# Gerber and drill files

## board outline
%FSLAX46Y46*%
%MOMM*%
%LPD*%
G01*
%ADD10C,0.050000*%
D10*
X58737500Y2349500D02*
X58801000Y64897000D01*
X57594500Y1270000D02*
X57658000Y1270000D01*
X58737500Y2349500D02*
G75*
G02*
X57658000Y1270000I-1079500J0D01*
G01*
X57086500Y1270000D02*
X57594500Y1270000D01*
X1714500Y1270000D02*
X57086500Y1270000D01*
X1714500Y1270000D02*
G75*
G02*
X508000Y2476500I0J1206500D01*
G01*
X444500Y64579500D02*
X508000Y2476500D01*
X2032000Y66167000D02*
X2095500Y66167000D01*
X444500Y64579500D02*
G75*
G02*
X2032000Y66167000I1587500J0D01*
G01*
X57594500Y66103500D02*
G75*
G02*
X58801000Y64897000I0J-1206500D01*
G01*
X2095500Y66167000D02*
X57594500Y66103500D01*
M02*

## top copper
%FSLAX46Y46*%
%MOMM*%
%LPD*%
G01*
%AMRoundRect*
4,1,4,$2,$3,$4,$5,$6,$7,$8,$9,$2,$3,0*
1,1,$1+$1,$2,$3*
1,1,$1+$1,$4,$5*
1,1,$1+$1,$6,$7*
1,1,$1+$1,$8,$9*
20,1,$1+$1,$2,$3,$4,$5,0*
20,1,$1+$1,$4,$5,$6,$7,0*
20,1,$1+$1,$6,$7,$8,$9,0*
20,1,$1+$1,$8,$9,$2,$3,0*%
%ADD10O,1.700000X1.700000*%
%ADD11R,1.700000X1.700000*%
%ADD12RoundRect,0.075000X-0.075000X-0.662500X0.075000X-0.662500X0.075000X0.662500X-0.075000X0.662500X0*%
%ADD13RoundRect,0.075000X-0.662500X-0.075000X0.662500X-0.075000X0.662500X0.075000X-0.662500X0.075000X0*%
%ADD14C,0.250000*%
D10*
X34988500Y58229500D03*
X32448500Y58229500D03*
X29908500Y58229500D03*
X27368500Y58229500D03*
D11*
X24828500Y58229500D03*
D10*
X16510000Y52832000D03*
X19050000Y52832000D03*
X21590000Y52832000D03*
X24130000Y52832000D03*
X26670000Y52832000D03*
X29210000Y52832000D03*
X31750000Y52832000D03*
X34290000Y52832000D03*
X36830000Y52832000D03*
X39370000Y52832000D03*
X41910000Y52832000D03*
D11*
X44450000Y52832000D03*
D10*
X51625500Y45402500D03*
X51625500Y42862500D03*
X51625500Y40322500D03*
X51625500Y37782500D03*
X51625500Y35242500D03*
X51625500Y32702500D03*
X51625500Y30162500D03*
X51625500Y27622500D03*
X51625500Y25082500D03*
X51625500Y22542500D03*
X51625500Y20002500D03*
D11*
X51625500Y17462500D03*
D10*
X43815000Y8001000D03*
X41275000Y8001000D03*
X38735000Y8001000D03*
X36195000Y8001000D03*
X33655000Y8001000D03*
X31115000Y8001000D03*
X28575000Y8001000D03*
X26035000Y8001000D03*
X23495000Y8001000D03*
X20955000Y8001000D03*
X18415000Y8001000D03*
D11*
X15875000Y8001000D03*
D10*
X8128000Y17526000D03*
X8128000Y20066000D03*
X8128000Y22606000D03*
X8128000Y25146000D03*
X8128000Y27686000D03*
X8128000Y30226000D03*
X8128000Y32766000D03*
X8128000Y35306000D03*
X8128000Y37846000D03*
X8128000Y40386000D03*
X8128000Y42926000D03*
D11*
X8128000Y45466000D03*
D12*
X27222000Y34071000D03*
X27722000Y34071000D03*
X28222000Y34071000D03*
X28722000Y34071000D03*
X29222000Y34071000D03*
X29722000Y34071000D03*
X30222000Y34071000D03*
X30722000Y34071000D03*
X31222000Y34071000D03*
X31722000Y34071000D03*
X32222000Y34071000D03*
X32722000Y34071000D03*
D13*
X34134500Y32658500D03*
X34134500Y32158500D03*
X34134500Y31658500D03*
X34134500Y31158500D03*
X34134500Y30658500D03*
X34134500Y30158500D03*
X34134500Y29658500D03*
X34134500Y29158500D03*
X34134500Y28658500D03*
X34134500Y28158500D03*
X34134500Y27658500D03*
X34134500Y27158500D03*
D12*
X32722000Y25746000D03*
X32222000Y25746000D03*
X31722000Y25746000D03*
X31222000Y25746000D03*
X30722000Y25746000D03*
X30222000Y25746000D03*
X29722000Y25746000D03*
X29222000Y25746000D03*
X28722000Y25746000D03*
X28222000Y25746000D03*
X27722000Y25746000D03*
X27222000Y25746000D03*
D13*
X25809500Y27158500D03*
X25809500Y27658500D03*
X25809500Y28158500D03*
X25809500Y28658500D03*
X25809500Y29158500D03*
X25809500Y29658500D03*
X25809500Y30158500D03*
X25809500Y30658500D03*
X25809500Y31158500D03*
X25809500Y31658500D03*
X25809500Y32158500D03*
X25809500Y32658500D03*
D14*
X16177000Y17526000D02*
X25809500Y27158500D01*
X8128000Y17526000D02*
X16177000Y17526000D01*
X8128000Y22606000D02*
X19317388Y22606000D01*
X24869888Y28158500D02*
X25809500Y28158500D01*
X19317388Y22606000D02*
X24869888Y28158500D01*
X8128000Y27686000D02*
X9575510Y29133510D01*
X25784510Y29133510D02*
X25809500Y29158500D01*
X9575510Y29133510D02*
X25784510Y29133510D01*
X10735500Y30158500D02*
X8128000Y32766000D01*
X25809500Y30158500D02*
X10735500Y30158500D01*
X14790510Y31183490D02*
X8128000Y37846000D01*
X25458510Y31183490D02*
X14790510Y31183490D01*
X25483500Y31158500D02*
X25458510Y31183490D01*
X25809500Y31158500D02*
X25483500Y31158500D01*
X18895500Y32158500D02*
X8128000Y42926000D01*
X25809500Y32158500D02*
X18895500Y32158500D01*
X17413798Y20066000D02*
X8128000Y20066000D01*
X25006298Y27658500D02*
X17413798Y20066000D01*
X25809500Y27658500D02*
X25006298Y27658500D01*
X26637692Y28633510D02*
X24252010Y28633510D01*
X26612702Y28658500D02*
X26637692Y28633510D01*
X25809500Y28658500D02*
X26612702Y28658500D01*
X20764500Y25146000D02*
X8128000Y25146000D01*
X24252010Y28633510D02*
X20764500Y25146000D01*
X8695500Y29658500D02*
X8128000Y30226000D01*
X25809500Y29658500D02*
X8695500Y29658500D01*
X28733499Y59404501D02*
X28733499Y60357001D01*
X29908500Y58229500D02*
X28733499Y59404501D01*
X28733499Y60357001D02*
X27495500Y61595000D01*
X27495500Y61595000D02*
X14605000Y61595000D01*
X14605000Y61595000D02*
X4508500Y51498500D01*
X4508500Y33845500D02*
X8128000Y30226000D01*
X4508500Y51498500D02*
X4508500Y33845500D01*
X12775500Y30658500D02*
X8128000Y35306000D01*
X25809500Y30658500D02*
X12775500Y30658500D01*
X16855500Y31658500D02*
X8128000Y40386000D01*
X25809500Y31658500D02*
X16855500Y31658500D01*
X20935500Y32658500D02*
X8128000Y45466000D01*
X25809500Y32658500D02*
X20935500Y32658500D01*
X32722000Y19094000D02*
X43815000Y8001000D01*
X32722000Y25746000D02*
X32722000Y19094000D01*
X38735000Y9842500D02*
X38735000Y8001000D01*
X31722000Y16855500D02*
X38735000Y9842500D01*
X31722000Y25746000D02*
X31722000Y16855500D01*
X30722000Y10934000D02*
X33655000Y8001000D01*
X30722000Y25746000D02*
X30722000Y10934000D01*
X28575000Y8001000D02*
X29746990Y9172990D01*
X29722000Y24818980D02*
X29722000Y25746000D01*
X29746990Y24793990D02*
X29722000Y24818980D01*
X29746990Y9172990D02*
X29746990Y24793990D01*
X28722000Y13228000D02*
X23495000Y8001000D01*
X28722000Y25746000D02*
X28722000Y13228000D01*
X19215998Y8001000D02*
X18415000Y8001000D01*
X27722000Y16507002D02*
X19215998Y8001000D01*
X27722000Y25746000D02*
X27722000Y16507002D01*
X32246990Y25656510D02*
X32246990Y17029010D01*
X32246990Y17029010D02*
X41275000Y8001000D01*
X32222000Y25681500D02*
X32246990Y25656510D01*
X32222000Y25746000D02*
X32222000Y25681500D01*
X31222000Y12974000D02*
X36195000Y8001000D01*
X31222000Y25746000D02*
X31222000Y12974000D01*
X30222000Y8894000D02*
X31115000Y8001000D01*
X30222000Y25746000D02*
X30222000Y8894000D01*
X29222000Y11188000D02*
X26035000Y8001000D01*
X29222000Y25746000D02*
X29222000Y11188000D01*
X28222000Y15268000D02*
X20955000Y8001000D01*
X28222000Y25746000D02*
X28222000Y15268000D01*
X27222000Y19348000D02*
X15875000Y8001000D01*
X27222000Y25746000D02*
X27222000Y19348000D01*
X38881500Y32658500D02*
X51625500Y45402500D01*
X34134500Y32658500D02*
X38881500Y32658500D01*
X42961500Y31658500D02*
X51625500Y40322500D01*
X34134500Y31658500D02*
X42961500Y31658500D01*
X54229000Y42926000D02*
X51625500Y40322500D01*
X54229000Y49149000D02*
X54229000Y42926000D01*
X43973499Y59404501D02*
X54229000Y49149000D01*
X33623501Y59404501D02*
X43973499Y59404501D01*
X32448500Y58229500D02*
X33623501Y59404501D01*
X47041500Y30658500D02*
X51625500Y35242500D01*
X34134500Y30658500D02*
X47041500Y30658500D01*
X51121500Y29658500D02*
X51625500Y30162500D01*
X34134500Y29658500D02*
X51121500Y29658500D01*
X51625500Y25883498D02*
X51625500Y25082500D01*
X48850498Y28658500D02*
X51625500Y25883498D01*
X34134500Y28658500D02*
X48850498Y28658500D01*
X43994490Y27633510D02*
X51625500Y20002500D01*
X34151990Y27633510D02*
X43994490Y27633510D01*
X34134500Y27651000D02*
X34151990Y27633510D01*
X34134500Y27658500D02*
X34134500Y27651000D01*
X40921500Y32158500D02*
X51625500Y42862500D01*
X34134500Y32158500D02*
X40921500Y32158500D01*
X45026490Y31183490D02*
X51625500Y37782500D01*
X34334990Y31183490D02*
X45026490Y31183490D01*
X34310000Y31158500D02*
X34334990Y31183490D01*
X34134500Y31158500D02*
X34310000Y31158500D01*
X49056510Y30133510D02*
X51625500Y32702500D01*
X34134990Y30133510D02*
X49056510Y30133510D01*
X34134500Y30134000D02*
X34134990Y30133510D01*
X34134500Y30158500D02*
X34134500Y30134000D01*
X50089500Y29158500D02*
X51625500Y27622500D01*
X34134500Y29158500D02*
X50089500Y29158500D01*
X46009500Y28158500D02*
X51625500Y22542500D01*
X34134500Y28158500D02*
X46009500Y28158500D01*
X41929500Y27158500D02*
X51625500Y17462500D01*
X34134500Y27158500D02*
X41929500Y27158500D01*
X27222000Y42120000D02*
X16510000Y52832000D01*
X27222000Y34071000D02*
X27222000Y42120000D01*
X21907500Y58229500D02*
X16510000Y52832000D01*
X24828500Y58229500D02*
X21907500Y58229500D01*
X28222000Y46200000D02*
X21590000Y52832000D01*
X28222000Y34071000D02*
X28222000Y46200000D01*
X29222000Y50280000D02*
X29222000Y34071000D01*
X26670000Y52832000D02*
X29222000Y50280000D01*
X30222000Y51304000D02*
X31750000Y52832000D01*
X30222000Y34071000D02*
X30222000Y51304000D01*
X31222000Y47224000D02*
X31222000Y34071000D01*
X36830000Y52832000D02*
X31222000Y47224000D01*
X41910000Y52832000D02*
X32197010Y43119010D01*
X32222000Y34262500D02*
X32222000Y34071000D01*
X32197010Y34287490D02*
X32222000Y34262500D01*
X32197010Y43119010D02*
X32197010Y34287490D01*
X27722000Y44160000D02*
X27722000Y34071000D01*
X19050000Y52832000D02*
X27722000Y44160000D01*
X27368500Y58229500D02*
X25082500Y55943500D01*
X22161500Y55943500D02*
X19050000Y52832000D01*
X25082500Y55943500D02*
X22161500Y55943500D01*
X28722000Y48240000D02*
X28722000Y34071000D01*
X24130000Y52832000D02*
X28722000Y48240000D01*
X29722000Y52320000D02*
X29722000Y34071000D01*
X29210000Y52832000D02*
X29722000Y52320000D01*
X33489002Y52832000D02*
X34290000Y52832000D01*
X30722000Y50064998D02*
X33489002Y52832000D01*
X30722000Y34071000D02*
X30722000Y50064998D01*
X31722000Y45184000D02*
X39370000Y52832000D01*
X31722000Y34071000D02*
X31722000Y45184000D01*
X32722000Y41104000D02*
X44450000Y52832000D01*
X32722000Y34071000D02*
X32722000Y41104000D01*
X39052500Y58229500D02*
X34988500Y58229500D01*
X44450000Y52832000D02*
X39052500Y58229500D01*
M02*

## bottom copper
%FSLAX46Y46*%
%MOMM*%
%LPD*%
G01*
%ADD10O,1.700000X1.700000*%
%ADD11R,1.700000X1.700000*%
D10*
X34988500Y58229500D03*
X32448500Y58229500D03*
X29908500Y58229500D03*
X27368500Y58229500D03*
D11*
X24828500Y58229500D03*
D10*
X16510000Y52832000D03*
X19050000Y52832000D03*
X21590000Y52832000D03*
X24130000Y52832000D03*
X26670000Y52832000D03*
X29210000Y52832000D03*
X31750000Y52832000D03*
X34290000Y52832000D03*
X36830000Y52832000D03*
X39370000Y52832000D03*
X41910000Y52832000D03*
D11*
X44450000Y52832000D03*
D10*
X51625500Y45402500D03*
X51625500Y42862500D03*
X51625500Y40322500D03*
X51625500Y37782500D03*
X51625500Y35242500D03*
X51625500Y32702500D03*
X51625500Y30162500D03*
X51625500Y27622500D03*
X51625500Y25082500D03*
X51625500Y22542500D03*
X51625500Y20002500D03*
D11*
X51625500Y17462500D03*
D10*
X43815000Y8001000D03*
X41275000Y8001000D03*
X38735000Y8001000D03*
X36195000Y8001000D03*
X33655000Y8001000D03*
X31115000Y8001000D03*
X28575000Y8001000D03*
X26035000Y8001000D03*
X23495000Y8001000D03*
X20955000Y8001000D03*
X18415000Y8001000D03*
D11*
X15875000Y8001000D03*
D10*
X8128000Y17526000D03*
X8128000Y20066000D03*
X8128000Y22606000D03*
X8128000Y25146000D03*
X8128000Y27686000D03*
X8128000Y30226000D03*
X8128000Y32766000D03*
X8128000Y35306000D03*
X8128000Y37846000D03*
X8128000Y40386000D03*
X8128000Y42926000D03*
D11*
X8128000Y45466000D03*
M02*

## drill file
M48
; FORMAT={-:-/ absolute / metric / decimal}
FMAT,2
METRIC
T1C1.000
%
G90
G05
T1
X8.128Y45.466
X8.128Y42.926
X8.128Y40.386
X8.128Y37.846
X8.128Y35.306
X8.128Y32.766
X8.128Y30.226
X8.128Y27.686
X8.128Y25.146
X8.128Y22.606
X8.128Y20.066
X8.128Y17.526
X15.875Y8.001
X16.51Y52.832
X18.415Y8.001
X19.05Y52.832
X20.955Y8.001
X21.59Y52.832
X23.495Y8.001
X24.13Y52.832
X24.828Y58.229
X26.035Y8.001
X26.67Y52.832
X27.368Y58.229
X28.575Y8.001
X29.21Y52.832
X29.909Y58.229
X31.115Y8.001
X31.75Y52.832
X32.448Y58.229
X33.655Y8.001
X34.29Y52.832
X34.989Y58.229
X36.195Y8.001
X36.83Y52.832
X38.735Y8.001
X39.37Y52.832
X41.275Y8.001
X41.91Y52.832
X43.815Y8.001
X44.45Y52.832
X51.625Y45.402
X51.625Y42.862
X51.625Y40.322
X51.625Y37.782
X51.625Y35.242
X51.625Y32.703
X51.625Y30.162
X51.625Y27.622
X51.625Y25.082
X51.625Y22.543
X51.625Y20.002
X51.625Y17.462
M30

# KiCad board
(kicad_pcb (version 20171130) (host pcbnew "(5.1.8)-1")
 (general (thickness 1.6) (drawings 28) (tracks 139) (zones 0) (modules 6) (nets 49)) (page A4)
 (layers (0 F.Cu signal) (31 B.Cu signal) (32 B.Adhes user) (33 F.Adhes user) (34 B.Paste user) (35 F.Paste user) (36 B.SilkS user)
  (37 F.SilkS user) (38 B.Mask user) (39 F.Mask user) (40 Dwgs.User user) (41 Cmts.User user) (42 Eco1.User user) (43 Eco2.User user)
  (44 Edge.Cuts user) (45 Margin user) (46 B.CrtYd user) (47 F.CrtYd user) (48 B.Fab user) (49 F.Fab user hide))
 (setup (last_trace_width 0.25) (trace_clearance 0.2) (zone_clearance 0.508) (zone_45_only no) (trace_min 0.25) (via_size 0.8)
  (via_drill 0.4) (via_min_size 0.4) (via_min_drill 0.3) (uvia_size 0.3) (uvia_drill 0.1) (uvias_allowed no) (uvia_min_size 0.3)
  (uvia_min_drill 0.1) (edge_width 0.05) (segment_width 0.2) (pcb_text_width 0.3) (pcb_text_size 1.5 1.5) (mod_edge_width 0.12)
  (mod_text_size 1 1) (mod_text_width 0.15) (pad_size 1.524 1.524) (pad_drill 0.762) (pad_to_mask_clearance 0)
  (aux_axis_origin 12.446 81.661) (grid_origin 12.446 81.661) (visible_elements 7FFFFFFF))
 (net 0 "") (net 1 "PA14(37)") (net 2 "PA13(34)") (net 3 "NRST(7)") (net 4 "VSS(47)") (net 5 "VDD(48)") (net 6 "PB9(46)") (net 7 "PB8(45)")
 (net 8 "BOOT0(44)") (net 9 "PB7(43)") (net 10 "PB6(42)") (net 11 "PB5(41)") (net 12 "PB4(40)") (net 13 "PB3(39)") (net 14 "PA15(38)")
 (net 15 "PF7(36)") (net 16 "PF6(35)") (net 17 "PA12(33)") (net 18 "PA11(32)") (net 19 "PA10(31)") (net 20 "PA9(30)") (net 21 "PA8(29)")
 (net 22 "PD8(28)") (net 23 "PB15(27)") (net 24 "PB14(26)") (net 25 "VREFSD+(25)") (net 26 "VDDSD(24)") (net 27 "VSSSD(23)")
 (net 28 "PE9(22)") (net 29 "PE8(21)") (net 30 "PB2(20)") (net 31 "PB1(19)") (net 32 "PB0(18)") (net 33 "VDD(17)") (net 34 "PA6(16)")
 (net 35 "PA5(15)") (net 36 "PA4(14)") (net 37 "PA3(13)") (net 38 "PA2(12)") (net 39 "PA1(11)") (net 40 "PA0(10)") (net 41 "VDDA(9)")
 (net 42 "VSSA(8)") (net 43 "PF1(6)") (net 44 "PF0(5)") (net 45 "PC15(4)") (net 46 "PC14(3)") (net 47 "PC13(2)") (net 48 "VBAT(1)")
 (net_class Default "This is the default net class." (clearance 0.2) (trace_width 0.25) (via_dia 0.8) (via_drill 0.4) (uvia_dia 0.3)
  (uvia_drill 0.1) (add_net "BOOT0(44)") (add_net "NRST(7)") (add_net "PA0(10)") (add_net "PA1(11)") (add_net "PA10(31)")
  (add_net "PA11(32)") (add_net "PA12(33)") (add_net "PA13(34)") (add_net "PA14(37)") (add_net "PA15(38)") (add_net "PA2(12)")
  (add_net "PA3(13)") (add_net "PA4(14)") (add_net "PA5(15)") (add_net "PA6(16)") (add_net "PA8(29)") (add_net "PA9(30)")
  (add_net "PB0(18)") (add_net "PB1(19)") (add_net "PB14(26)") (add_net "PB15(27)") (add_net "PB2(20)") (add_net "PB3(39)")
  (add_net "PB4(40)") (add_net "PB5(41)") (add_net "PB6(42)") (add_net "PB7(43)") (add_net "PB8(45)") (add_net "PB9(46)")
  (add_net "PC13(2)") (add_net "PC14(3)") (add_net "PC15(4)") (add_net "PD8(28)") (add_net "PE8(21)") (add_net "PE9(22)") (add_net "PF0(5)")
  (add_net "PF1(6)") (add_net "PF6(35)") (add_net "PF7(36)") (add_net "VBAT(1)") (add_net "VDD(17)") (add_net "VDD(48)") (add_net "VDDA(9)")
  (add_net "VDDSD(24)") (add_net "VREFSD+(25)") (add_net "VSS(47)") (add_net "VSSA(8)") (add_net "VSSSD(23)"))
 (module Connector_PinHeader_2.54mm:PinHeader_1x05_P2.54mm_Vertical (layer F.Cu) (at 24.8285 -58.2295 90)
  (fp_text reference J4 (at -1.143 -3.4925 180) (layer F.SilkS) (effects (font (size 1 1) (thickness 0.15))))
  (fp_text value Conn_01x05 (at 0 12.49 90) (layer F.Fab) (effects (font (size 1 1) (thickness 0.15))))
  (pad 5 thru_hole oval (at 0 10.16 90) (size 1.7 1.7) (drill 1) (layers *.Cu *.Mask) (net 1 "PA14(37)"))
  (pad 4 thru_hole oval (at 0 7.62 90) (size 1.7 1.7) (drill 1) (layers *.Cu *.Mask) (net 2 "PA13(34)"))
  (pad 3 thru_hole oval (at 0 5.08 90) (size 1.7 1.7) (drill 1) (layers *.Cu *.Mask) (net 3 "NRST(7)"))
  (pad 2 thru_hole oval (at 0 2.54 90) (size 1.7 1.7) (drill 1) (layers *.Cu *.Mask) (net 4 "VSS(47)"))
  (pad 1 thru_hole rect (at 0 0 90) (size 1.7 1.7) (drill 1) (layers *.Cu *.Mask) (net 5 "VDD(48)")))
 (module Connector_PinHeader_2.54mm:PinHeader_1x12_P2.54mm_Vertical (layer F.Cu) (at 44.45 -52.832 270)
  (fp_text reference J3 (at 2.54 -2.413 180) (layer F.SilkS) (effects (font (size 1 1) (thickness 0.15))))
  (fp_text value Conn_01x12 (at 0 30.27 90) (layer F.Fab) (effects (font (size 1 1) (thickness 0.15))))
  (pad 12 thru_hole oval (at 0 27.94 270) (size 1.7 1.7) (drill 1) (layers *.Cu *.Mask) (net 5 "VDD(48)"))
  (pad 11 thru_hole oval (at 0 25.4 270) (size 1.7 1.7) (drill 1) (layers *.Cu *.Mask) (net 4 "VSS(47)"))
  (pad 10 thru_hole oval (at 0 22.86 270) (size 1.7 1.7) (drill 1) (layers *.Cu *.Mask) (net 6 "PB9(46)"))
  (pad 9 thru_hole oval (at 0 20.32 270) (size 1.7 1.7) (drill 1) (layers *.Cu *.Mask) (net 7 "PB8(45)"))
  (pad 8 thru_hole oval (at 0 17.78 270) (size 1.7 1.7) (drill 1) (layers *.Cu *.Mask) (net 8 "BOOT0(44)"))
  (pad 7 thru_hole oval (at 0 15.24 270) (size 1.7 1.7) (drill 1) (layers *.Cu *.Mask) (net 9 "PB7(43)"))
  (pad 6 thru_hole oval (at 0 12.7 270) (size 1.7 1.7) (drill 1) (layers *.Cu *.Mask) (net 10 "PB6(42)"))
  (pad 5 thru_hole oval (at 0 10.16 270) (size 1.7 1.7) (drill 1) (layers *.Cu *.Mask) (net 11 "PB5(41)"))
  (pad 4 thru_hole oval (at 0 7.62 270) (size 1.7 1.7) (drill 1) (layers *.Cu *.Mask) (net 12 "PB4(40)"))
  (pad 3 thru_hole oval (at 0 5.08 270) (size 1.7 1.7) (drill 1) (layers *.Cu *.Mask) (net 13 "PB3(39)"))
  (pad 2 thru_hole oval (at 0 2.54 270) (size 1.7 1.7) (drill 1) (layers *.Cu *.Mask) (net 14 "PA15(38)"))
  (pad 1 thru_hole rect (at 0 0 270) (size 1.7 1.7) (drill 1) (layers *.Cu *.Mask) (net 1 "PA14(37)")))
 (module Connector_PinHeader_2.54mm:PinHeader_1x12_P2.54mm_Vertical (layer F.Cu) (at 51.6255 -17.4625 180)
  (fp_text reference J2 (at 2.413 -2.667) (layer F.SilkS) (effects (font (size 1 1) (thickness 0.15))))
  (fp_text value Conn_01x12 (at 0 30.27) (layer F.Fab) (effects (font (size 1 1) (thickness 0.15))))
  (pad 12 thru_hole oval (at 0 27.94 180) (size 1.7 1.7) (drill 1) (layers *.Cu *.Mask) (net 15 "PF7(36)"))
  (pad 11 thru_hole oval (at 0 25.4 180) (size 1.7 1.7) (drill 1) (layers *.Cu *.Mask) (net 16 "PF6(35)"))
  (pad 10 thru_hole oval (at 0 22.86 180) (size 1.7 1.7) (drill 1) (layers *.Cu *.Mask) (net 2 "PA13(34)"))
  (pad 9 thru_hole oval (at 0 20.32 180) (size 1.7 1.7) (drill 1) (layers *.Cu *.Mask) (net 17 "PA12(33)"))
  (pad 8 thru_hole oval (at 0 17.78 180) (size 1.7 1.7) (drill 1) (layers *.Cu *.Mask) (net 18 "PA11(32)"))
  (pad 7 thru_hole oval (at 0 15.24 180) (size 1.7 1.7) (drill 1) (layers *.Cu *.Mask) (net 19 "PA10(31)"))
  (pad 6 thru_hole oval (at 0 12.7 180) (size 1.7 1.7) (drill 1) (layers *.Cu *.Mask) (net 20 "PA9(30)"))
  (pad 5 thru_hole oval (at 0 10.16 180) (size 1.7 1.7) (drill 1) (layers *.Cu *.Mask) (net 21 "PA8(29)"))
  (pad 4 thru_hole oval (at 0 7.62 180) (size 1.7 1.7) (drill 1) (layers *.Cu *.Mask) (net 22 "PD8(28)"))
  (pad 3 thru_hole oval (at 0 5.08 180) (size 1.7 1.7) (drill 1) (layers *.Cu *.Mask) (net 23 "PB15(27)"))
  (pad 2 thru_hole oval (at 0 2.54 180) (size 1.7 1.7) (drill 1) (layers *.Cu *.Mask) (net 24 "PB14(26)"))
  (pad 1 thru_hole rect (at 0 0 180) (size 1.7 1.7) (drill 1) (layers *.Cu *.Mask) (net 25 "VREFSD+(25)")))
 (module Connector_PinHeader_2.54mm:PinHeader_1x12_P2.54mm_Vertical (layer F.Cu) (at 15.875 -8.001 90)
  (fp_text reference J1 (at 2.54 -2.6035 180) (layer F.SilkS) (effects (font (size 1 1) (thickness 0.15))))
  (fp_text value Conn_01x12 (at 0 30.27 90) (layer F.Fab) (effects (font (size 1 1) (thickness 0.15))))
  (pad 12 thru_hole oval (at 0 27.94 90) (size 1.7 1.7) (drill 1) (layers *.Cu *.Mask) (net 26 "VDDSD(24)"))
  (pad 11 thru_hole oval (at 0 25.4 90) (size 1.7 1.7) (drill 1) (layers *.Cu *.Mask) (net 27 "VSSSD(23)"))
  (pad 10 thru_hole oval (at 0 22.86 90) (size 1.7 1.7) (drill 1) (layers *.Cu *.Mask) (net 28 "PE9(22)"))
  (pad 9 thru_hole oval (at 0 20.32 90) (size 1.7 1.7) (drill 1) (layers *.Cu *.Mask) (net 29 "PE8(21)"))
  (pad 8 thru_hole oval (at 0 17.78 90) (size 1.7 1.7) (drill 1) (layers *.Cu *.Mask) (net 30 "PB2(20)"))
  (pad 7 thru_hole oval (at 0 15.24 90) (size 1.7 1.7) (drill 1) (layers *.Cu *.Mask) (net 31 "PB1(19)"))
  (pad 6 thru_hole oval (at 0 12.7 90) (size 1.7 1.7) (drill 1) (layers *.Cu *.Mask) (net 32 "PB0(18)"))
  (pad 5 thru_hole oval (at 0 10.16 90) (size 1.7 1.7) (drill 1) (layers *.Cu *.Mask) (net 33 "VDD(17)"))
  (pad 4 thru_hole oval (at 0 7.62 90) (size 1.7 1.7) (drill 1) (layers *.Cu *.Mask) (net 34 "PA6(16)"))
  (pad 3 thru_hole oval (at 0 5.08 90) (size 1.7 1.7) (drill 1) (layers *.Cu *.Mask) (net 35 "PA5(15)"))
  (pad 2 thru_hole oval (at 0 2.54 90) (size 1.7 1.7) (drill 1) (layers *.Cu *.Mask) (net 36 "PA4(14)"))
  (pad 1 thru_hole rect (at 0 0 90) (size 1.7 1.7) (drill 1) (layers *.Cu *.Mask) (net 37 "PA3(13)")))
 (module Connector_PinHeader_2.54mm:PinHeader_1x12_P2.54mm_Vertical (layer F.Cu) (at 8.128 -45.466)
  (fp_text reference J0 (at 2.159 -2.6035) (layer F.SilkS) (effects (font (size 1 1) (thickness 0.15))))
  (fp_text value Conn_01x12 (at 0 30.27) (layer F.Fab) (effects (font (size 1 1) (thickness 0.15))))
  (pad 12 thru_hole oval (at 0 27.94) (size 1.7 1.7) (drill 1) (layers *.Cu *.Mask) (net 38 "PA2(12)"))
  (pad 11 thru_hole oval (at 0 25.4) (size 1.7 1.7) (drill 1) (layers *.Cu *.Mask) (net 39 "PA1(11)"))
  (pad 10 thru_hole oval (at 0 22.86) (size 1.7 1.7) (drill 1) (layers *.Cu *.Mask) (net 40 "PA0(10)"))
  (pad 9 thru_hole oval (at 0 20.32) (size 1.7 1.7) (drill 1) (layers *.Cu *.Mask) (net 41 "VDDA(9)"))
  (pad 8 thru_hole oval (at 0 17.78) (size 1.7 1.7) (drill 1) (layers *.Cu *.Mask) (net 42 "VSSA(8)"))
  (pad 7 thru_hole oval (at 0 15.24) (size 1.7 1.7) (drill 1) (layers *.Cu *.Mask) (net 3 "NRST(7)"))
  (pad 6 thru_hole oval (at 0 12.7) (size 1.7 1.7) (drill 1) (layers *.Cu *.Mask) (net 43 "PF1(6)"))
  (pad 5 thru_hole oval (at 0 10.16) (size 1.7 1.7) (drill 1) (layers *.Cu *.Mask) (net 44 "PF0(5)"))
  (pad 4 thru_hole oval (at 0 7.62) (size 1.7 1.7) (drill 1) (layers *.Cu *.Mask) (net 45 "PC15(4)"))
  (pad 3 thru_hole oval (at 0 5.08) (size 1.7 1.7) (drill 1) (layers *.Cu *.Mask) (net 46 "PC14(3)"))
  (pad 2 thru_hole oval (at 0 2.54) (size 1.7 1.7) (drill 1) (layers *.Cu *.Mask) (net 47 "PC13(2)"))
  (pad 1 thru_hole rect (at 0 0) (size 1.7 1.7) (drill 1) (layers *.Cu *.Mask) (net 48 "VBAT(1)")))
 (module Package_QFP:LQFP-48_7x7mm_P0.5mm (layer F.Cu) (at 29.972 -29.9085)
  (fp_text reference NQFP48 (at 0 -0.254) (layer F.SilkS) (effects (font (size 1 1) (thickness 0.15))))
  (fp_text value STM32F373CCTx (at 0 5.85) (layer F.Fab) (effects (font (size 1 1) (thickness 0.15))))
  (pad 48 smd roundrect (at -2.75 -4.1625) (size 0.3 1.475) (layers F.Cu F.Paste F.Mask) (roundrect_rratio 0.25) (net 5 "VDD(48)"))
  (pad 47 smd roundrect (at -2.25 -4.1625) (size 0.3 1.475) (layers F.Cu F.Paste F.Mask) (roundrect_rratio 0.25) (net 4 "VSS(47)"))
  (pad 46 smd roundrect (at -1.75 -4.1625) (size 0.3 1.475) (layers F.Cu F.Paste F.Mask) (roundrect_rratio 0.25) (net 6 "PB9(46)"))
  (pad 45 smd roundrect (at -1.25 -4.1625) (size 0.3 1.475) (layers F.Cu F.Paste F.Mask) (roundrect_rratio 0.25) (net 7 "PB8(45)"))
  (pad 44 smd roundrect (at -0.75 -4.1625) (size 0.3 1.475) (layers F.Cu F.Paste F.Mask) (roundrect_rratio 0.25) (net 8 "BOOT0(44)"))
  (pad 43 smd roundrect (at -0.25 -4.1625) (size 0.3 1.475) (layers F.Cu F.Paste F.Mask) (roundrect_rratio 0.25) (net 9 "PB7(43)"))
  (pad 42 smd roundrect (at 0.25 -4.1625) (size 0.3 1.475) (layers F.Cu F.Paste F.Mask) (roundrect_rratio 0.25) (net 10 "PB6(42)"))
  (pad 41 smd roundrect (at 0.75 -4.1625) (size 0.3 1.475) (layers F.Cu F.Paste F.Mask) (roundrect_rratio 0.25) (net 11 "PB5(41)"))
  (pad 40 smd roundrect (at 1.25 -4.1625) (size 0.3 1.475) (layers F.Cu F.Paste F.Mask) (roundrect_rratio 0.25) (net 12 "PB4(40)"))
  (pad 39 smd roundrect (at 1.75 -4.1625) (size 0.3 1.475) (layers F.Cu F.Paste F.Mask) (roundrect_rratio 0.25) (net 13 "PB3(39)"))
  (pad 38 smd roundrect (at 2.25 -4.1625) (size 0.3 1.475) (layers F.Cu F.Paste F.Mask) (roundrect_rratio 0.25) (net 14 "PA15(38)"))
  (pad 37 smd roundrect (at 2.75 -4.1625) (size 0.3 1.475) (layers F.Cu F.Paste F.Mask) (roundrect_rratio 0.25) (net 1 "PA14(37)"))
  (pad 36 smd roundrect (at 4.1625 -2.75) (size 1.475 0.3) (layers F.Cu F.Paste F.Mask) (roundrect_rratio 0.25) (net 15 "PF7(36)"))
  (pad 35 smd roundrect (at 4.1625 -2.25) (size 1.475 0.3) (layers F.Cu F.Paste F.Mask) (roundrect_rratio 0.25) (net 16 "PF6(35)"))
  (pad 34 smd roundrect (at 4.1625 -1.75) (size 1.475 0.3) (layers F.Cu F.Paste F.Mask) (roundrect_rratio 0.25) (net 2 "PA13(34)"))
  (pad 33 smd roundrect (at 4.1625 -1.25) (size 1.475 0.3) (layers F.Cu F.Paste F.Mask) (roundrect_rratio 0.25) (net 17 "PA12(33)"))
  (pad 32 smd roundrect (at 4.1625 -0.75) (size 1.475 0.3) (layers F.Cu F.Paste F.Mask) (roundrect_rratio 0.25) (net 18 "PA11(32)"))
  (pad 31 smd roundrect (at 4.1625 -0.25) (size 1.475 0.3) (layers F.Cu F.Paste F.Mask) (roundrect_rratio 0.25) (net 19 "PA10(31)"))
  (pad 30 smd roundrect (at 4.1625 0.25) (size 1.475 0.3) (layers F.Cu F.Paste F.Mask) (roundrect_rratio 0.25) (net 20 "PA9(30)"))
  (pad 29 smd roundrect (at 4.1625 0.75) (size 1.475 0.3) (layers F.Cu F.Paste F.Mask) (roundrect_rratio 0.25) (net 21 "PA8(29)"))
  (pad 28 smd roundrect (at 4.1625 1.25) (size 1.475 0.3) (layers F.Cu F.Paste F.Mask) (roundrect_rratio 0.25) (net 22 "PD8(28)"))
  (pad 27 smd roundrect (at 4.1625 1.75) (size 1.475 0.3) (layers F.Cu F.Paste F.Mask) (roundrect_rratio 0.25) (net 23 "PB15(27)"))
  (pad 26 smd roundrect (at 4.1625 2.25) (size 1.475 0.3) (layers F.Cu F.Paste F.Mask) (roundrect_rratio 0.25) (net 24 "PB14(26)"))
  (pad 25 smd roundrect (at 4.1625 2.75) (size 1.475 0.3) (layers F.Cu F.Paste F.Mask) (roundrect_rratio 0.25) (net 25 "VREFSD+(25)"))
  (pad 24 smd roundrect (at 2.75 4.1625) (size 0.3 1.475) (layers F.Cu F.Paste F.Mask) (roundrect_rratio 0.25) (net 26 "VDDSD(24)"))
  (pad 23 smd roundrect (at 2.25 4.1625) (size 0.3 1.475) (layers F.Cu F.Paste F.Mask) (roundrect_rratio 0.25) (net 27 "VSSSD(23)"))
  (pad 22 smd roundrect (at 1.75 4.1625) (size 0.3 1.475) (layers F.Cu F.Paste F.Mask) (roundrect_rratio 0.25) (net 28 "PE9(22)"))
  (pad 21 smd roundrect (at 1.25 4.1625) (size 0.3 1.475) (layers F.Cu F.Paste F.Mask) (roundrect_rratio 0.25) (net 29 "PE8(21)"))
  (pad 20 smd roundrect (at 0.75 4.1625) (size 0.3 1.475) (layers F.Cu F.Paste F.Mask) (roundrect_rratio 0.25) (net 30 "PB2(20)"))
  (pad 19 smd roundrect (at 0.25 4.1625) (size 0.3 1.475) (layers F.Cu F.Paste F.Mask) (roundrect_rratio 0.25) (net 31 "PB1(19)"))
  (pad 18 smd roundrect (at -0.25 4.1625) (size 0.3 1.475) (layers F.Cu F.Paste F.Mask) (roundrect_rratio 0.25) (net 32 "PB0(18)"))
  (pad 17 smd roundrect (at -0.75 4.1625) (size 0.3 1.475) (layers F.Cu F.Paste F.Mask) (roundrect_rratio 0.25) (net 33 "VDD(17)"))
  (pad 16 smd roundrect (at -1.25 4.1625) (size 0.3 1.475) (layers F.Cu F.Paste F.Mask) (roundrect_rratio 0.25) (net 34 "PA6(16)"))
  (pad 15 smd roundrect (at -1.75 4.1625) (size 0.3 1.475) (layers F.Cu F.Paste F.Mask) (roundrect_rratio 0.25) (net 35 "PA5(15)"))
  (pad 14 smd roundrect (at -2.25 4.1625) (size 0.3 1.475) (layers F.Cu F.Paste F.Mask) (roundrect_rratio 0.25) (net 36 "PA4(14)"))
  (pad 13 smd roundrect (at -2.75 4.1625) (size 0.3 1.475) (layers F.Cu F.Paste F.Mask) (roundrect_rratio 0.25) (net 37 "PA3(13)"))
  (pad 12 smd roundrect (at -4.1625 2.75) (size 1.475 0.3) (layers F.Cu F.Paste F.Mask) (roundrect_rratio 0.25) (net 38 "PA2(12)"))
  (pad 11 smd roundrect (at -4.1625 2.25) (size 1.475 0.3) (layers F.Cu F.Paste F.Mask) (roundrect_rratio 0.25) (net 39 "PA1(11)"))
  (pad 10 smd roundrect (at -4.1625 1.75) (size 1.475 0.3) (layers F.Cu F.Paste F.Mask) (roundrect_rratio 0.25) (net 40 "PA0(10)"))
  (pad 9 smd roundrect (at -4.1625 1.25) (size 1.475 0.3) (layers F.Cu F.Paste F.Mask) (roundrect_rratio 0.25) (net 41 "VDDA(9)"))
  (pad 8 smd roundrect (at -4.1625 0.75) (size 1.475 0.3) (layers F.Cu F.Paste F.Mask) (roundrect_rratio 0.25) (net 42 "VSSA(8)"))
  (pad 7 smd roundrect (at -4.1625 0.25) (size 1.475 0.3) (layers F.Cu F.Paste F.Mask) (roundrect_rratio 0.25) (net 3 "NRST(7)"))
  (pad 6 smd roundrect (at -4.1625 -0.25) (size 1.475 0.3) (layers F.Cu F.Paste F.Mask) (roundrect_rratio 0.25) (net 43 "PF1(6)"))
  (pad 5 smd roundrect (at -4.1625 -0.75) (size 1.475 0.3) (layers F.Cu F.Paste F.Mask) (roundrect_rratio 0.25) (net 44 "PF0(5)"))
  (pad 4 smd roundrect (at -4.1625 -1.25) (size 1.475 0.3) (layers F.Cu F.Paste F.Mask) (roundrect_rratio 0.25) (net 45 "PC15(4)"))
  (pad 3 smd roundrect (at -4.1625 -1.75) (size 1.475 0.3) (layers F.Cu F.Paste F.Mask) (roundrect_rratio 0.25) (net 46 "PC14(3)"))
  (pad 2 smd roundrect (at -4.1625 -2.25) (size 1.475 0.3) (layers F.Cu F.Paste F.Mask) (roundrect_rratio 0.25) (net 47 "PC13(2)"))
  (pad 1 smd roundrect (at -4.1625 -2.75) (size 1.475 0.3) (layers F.Cu F.Paste F.Mask) (roundrect_rratio 0.25) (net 48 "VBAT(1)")))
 (gr_line (start 58.7375 -2.3495) (end 58.801 -64.897) (layer Edge.Cuts) (width 0.05))
 (gr_line (start 57.5945 -1.27) (end 57.658 -1.27) (layer Edge.Cuts) (width 0.05))
 (gr_arc (start 57.658 -2.3495) (end 57.658 -1.27) (angle -90) (layer Edge.Cuts) (width 0.05))
 (gr_line (start 57.0865 -1.27) (end 57.5945 -1.27) (layer Edge.Cuts) (width 0.05))
 (gr_line (start 1.7145 -1.27) (end 57.0865 -1.27) (layer Edge.Cuts) (width 0.05))
 (gr_arc (start 1.7145 -2.4765) (end 0.508 -2.4765) (angle -90) (layer Edge.Cuts) (width 0.05))
 (gr_line (start 0.4445 -64.5795) (end 0.508 -2.4765) (layer Edge.Cuts) (width 0.05))
 (gr_line (start 2.032 -66.167) (end 2.0955 -66.167) (layer Edge.Cuts) (width 0.05))
 (gr_arc (start 2.032 -64.5795) (end 2.032 -66.167) (angle -90) (layer Edge.Cuts) (width 0.05))
 (gr_arc (start 57.5945 -64.897) (end 58.801 -64.897) (angle -90) (layer Edge.Cuts) (width 0.05))
 (gr_line (start 2.0955 -66.167) (end 57.5945 -66.1035) (layer Edge.Cuts) (width 0.05))
 (segment (start 16.177 -17.526) (end 25.8095 -27.1585) (width 0.25) (layer F.Cu) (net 38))
 (segment (start 8.128 -17.526) (end 16.177 -17.526) (width 0.25) (layer F.Cu) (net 38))
 (segment (start 8.128 -22.606) (end 19.317388 -22.606) (width 0.25) (layer F.Cu) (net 40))
 (segment (start 24.869888 -28.1585) (end 25.8095 -28.1585) (width 0.25) (layer F.Cu) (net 40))
 (segment (start 19.317388 -22.606) (end 24.869888 -28.1585) (width 0.25) (layer F.Cu) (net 40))
 (segment (start 8.128 -27.686) (end 9.57551 -29.13351) (width 0.25) (layer F.Cu) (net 42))
 (segment (start 25.78451 -29.13351) (end 25.8095 -29.1585) (width 0.25) (layer F.Cu) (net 42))
 (segment (start 9.57551 -29.13351) (end 25.78451 -29.13351) (width 0.25) (layer F.Cu) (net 42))
 (segment (start 10.7355 -30.1585) (end 8.128 -32.766) (width 0.25) (layer F.Cu) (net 43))
 (segment (start 25.8095 -30.1585) (end 10.7355 -30.1585) (width 0.25) (layer F.Cu) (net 43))
 (segment (start 14.79051 -31.18349) (end 8.128 -37.846) (width 0.25) (layer F.Cu) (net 45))
 (segment (start 25.45851 -31.18349) (end 14.79051 -31.18349) (width 0.25) (layer F.Cu) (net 45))
 (segment (start 25.4835 -31.1585) (end 25.45851 -31.18349) (width 0.25) (layer F.Cu) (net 45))
 (segment (start 25.8095 -31.1585) (end 25.4835 -31.1585) (width 0.25) (layer F.Cu) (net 45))
 (segment (start 18.8955 -32.1585) (end 8.128 -42.926) (width 0.25) (layer F.Cu) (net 47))
 (segment (start 25.8095 -32.1585) (end 18.8955 -32.1585) (width 0.25) (layer F.Cu) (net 47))
 (segment (start 17.413798 -20.066) (end 8.128 -20.066) (width 0.25) (layer F.Cu) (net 39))
 (segment (start 25.006298 -27.6585) (end 17.413798 -20.066) (width 0.25) (layer F.Cu) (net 39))
 (segment (start 25.8095 -27.6585) (end 25.006298 -27.6585) (width 0.25) (layer F.Cu) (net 39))
 (segment (start 26.637692 -28.63351) (end 24.25201 -28.63351) (width 0.25) (layer F.Cu) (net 41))
 (segment (start 26.612702 -28.6585) (end 26.637692 -28.63351) (width 0.25) (layer F.Cu) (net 41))
 (segment (start 25.8095 -28.6585) (end 26.612702 -28.6585) (width 0.25) (layer F.Cu) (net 41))
 (segment (start 20.7645 -25.146) (end 8.128 -25.146) (width 0.25) (layer F.Cu) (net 41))
 (segment (start 24.25201 -28.63351) (end 20.7645 -25.146) (width 0.25) (layer F.Cu) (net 41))
 (segment (start 8.6955 -29.6585) (end 8.128 -30.226) (width 0.25) (layer F.Cu) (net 3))
 (segment (start 25.8095 -29.6585) (end 8.6955 -29.6585) (width 0.25) (layer F.Cu) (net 3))
 (segment (start 28.733499 -59.404501) (end 28.733499 -60.357001) (width 0.25) (layer F.Cu) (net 3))
 (segment (start 29.9085 -58.2295) (end 28.733499 -59.404501) (width 0.25) (layer F.Cu) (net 3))
 (segment (start 28.733499 -60.357001) (end 27.4955 -61.595) (width 0.25) (layer F.Cu) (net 3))
 (segment (start 27.4955 -61.595) (end 14.605 -61.595) (width 0.25) (layer F.Cu) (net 3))
 (segment (start 14.605 -61.595) (end 4.5085 -51.4985) (width 0.25) (layer F.Cu) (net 3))
 (segment (start 4.5085 -33.8455) (end 8.128 -30.226) (width 0.25) (layer F.Cu) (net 3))
 (segment (start 4.5085 -51.4985) (end 4.5085 -33.8455) (width 0.25) (layer F.Cu) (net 3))
 (segment (start 12.7755 -30.6585) (end 8.128 -35.306) (width 0.25) (layer F.Cu) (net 44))
 (segment (start 25.8095 -30.6585) (end 12.7755 -30.6585) (width 0.25) (layer F.Cu) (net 44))
 (segment (start 16.8555 -31.6585) (end 8.128 -40.386) (width 0.25) (layer F.Cu) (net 46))
 (segment (start 25.8095 -31.6585) (end 16.8555 -31.6585) (width 0.25) (layer F.Cu) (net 46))
 (segment (start 20.9355 -32.6585) (end 8.128 -45.466) (width 0.25) (layer F.Cu) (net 48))
 (segment (start 25.8095 -32.6585) (end 20.9355 -32.6585) (width 0.25) (layer F.Cu) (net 48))
 (segment (start 32.722 -19.094) (end 43.815 -8.001) (width 0.25) (layer F.Cu) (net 26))
 (segment (start 32.722 -25.746) (end 32.722 -19.094) (width 0.25) (layer F.Cu) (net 26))
 (segment (start 38.735 -9.8425) (end 38.735 -8.001) (width 0.25) (layer F.Cu) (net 28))
 (segment (start 31.722 -16.8555) (end 38.735 -9.8425) (width 0.25) (layer F.Cu) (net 28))
 (segment (start 31.722 -25.746) (end 31.722 -16.8555) (width 0.25) (layer F.Cu) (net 28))
 (segment (start 30.722 -10.934) (end 33.655 -8.001) (width 0.25) (layer F.Cu) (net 30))
 (segment (start 30.722 -25.746) (end 30.722 -10.934) (width 0.25) (layer F.Cu) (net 30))
 (segment (start 28.575 -8.001) (end 29.74699 -9.17299) (width 0.25) (layer F.Cu) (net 32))
 (segment (start 29.722 -24.81898) (end 29.722 -25.746) (width 0.25) (layer F.Cu) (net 32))
 (segment (start 29.74699 -24.79399) (end 29.722 -24.81898) (width 0.25) (layer F.Cu) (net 32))
 (segment (start 29.74699 -9.17299) (end 29.74699 -24.79399) (width 0.25) (layer F.Cu) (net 32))
 (segment (start 28.722 -13.228) (end 23.495 -8.001) (width 0.25) (layer F.Cu) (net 34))
 (segment (start 28.722 -25.746) (end 28.722 -13.228) (width 0.25) (layer F.Cu) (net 34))
 (segment (start 19.215998 -8.001) (end 18.415 -8.001) (width 0.25) (layer F.Cu) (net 36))
 (segment (start 27.722 -16.507002) (end 19.215998 -8.001) (width 0.25) (layer F.Cu) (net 36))
 (segment (start 27.722 -25.746) (end 27.722 -16.507002) (width 0.25) (layer F.Cu) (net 36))
 (segment (start 32.24699 -25.65651) (end 32.24699 -17.02901) (width 0.25) (layer F.Cu) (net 27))
 (segment (start 32.24699 -17.02901) (end 41.275 -8.001) (width 0.25) (layer F.Cu) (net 27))
 (segment (start 32.222 -25.6815) (end 32.24699 -25.65651) (width 0.25) (layer F.Cu) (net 27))
 (segment (start 32.222 -25.746) (end 32.222 -25.6815) (width 0.25) (layer F.Cu) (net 27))
 (segment (start 31.222 -12.974) (end 36.195 -8.001) (width 0.25) (layer F.Cu) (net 29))
 (segment (start 31.222 -25.746) (end 31.222 -12.974) (width 0.25) (layer F.Cu) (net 29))
 (segment (start 30.222 -8.894) (end 31.115 -8.001) (width 0.25) (layer F.Cu) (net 31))
 (segment (start 30.222 -25.746) (end 30.222 -8.894) (width 0.25) (layer F.Cu) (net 31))
 (segment (start 29.222 -11.188) (end 26.035 -8.001) (width 0.25) (layer F.Cu) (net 33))
 (segment (start 29.222 -25.746) (end 29.222 -11.188) (width 0.25) (layer F.Cu) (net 33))
 (segment (start 28.222 -15.268) (end 20.955 -8.001) (width 0.25) (layer F.Cu) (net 35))
 (segment (start 28.222 -25.746) (end 28.222 -15.268) (width 0.25) (layer F.Cu) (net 35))
 (segment (start 27.222 -19.348) (end 15.875 -8.001) (width 0.25) (layer F.Cu) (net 37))
 (segment (start 27.222 -25.746) (end 27.222 -19.348) (width 0.25) (layer F.Cu) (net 37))
 (segment (start 38.8815 -32.6585) (end 51.6255 -45.4025) (width 0.25) (layer F.Cu) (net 15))
 (segment (start 34.1345 -32.6585) (end 38.8815 -32.6585) (width 0.25) (layer F.Cu) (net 15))
 (segment (start 42.9615 -31.6585) (end 51.6255 -40.3225) (width 0.25) (layer F.Cu) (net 2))
 (segment (start 34.1345 -31.6585) (end 42.9615 -31.6585) (width 0.25) (layer F.Cu) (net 2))
 (segment (start 54.229 -42.926) (end 51.6255 -40.3225) (width 0.25) (layer F.Cu) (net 2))
 (segment (start 54.229 -49.149) (end 54.229 -42.926) (width 0.25) (layer F.Cu) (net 2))
 (segment (start 43.973499 -59.404501) (end 54.229 -49.149) (width 0.25) (layer F.Cu) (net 2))
 (segment (start 33.623501 -59.404501) (end 43.973499 -59.404501) (width 0.25) (layer F.Cu) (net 2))
 (segment (start 32.4485 -58.2295) (end 33.623501 -59.404501) (width 0.25) (layer F.Cu) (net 2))
 (segment (start 47.0415 -30.6585) (end 51.6255 -35.2425) (width 0.25) (layer F.Cu) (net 18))
 (segment (start 34.1345 -30.6585) (end 47.0415 -30.6585) (width 0.25) (layer F.Cu) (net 18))
 (segment (start 51.1215 -29.6585) (end 51.6255 -30.1625) (width 0.25) (layer F.Cu) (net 20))
 (segment (start 34.1345 -29.6585) (end 51.1215 -29.6585) (width 0.25) (layer F.Cu) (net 20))
 (segment (start 51.6255 -25.883498) (end 51.6255 -25.0825) (width 0.25) (layer F.Cu) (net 22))
 (segment (start 48.850498 -28.6585) (end 51.6255 -25.883498) (width 0.25) (layer F.Cu) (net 22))
 (segment (start 34.1345 -28.6585) (end 48.850498 -28.6585) (width 0.25) (layer F.Cu) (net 22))
 (segment (start 43.99449 -27.63351) (end 51.6255 -20.0025) (width 0.25) (layer F.Cu) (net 24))
 (segment (start 34.15199 -27.63351) (end 43.99449 -27.63351) (width 0.25) (layer F.Cu) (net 24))
 (segment (start 34.1345 -27.651) (end 34.15199 -27.63351) (width 0.25) (layer F.Cu) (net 24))
 (segment (start 34.1345 -27.6585) (end 34.1345 -27.651) (width 0.25) (layer F.Cu) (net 24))
 (segment (start 40.9215 -32.1585) (end 51.6255 -42.8625) (width 0.25) (layer F.Cu) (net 16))
 (segment (start 34.1345 -32.1585) (end 40.9215 -32.1585) (width 0.25) (layer F.Cu) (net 16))
 (segment (start 45.02649 -31.18349) (end 51.6255 -37.7825) (width 0.25) (layer F.Cu) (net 17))
 (segment (start 34.33499 -31.18349) (end 45.02649 -31.18349) (width 0.25) (layer F.Cu) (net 17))
 (segment (start 34.31 -31.1585) (end 34.33499 -31.18349) (width 0.25) (layer F.Cu) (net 17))
 (segment (start 34.1345 -31.1585) (end 34.31 -31.1585) (width 0.25) (layer F.Cu) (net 17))
 (segment (start 49.05651 -30.13351) (end 51.6255 -32.7025) (width 0.25) (layer F.Cu) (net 19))
 (segment (start 34.13499 -30.13351) (end 49.05651 -30.13351) (width 0.25) (layer F.Cu) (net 19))
 (segment (start 34.1345 -30.134) (end 34.13499 -30.13351) (width 0.25) (layer F.Cu) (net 19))
 (segment (start 34.1345 -30.1585) (end 34.1345 -30.134) (width 0.25) (layer F.Cu) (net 19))
 (segment (start 50.0895 -29.1585) (end 51.6255 -27.6225) (width 0.25) (layer F.Cu) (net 21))
 (segment (start 34.1345 -29.1585) (end 50.0895 -29.1585) (width 0.25) (layer F.Cu) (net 21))
 (segment (start 46.0095 -28.1585) (end 51.6255 -22.5425) (width 0.25) (layer F.Cu) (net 23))
 (segment (start 34.1345 -28.1585) (end 46.0095 -28.1585) (width 0.25) (layer F.Cu) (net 23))
 (segment (start 41.9295 -27.1585) (end 51.6255 -17.4625) (width 0.25) (layer F.Cu) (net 25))
 (segment (start 34.1345 -27.1585) (end 41.9295 -27.1585) (width 0.25) (layer F.Cu) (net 25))
 (segment (start 27.222 -42.12) (end 16.51 -52.832) (width 0.25) (layer F.Cu) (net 5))
 (segment (start 27.222 -34.071) (end 27.222 -42.12) (width 0.25) (layer F.Cu) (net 5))
 (segment (start 21.9075 -58.2295) (end 16.51 -52.832) (width 0.25) (layer F.Cu) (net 5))
 (segment (start 24.8285 -58.2295) (end 21.9075 -58.2295) (width 0.25) (layer F.Cu) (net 5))
 (segment (start 28.222 -46.2) (end 21.59 -52.832) (width 0.25) (layer F.Cu) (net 6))
 (segment (start 28.222 -34.071) (end 28.222 -46.2) (width 0.25) (layer F.Cu) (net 6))
 (segment (start 29.222 -50.28) (end 29.222 -34.071) (width 0.25) (layer F.Cu) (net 8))
 (segment (start 26.67 -52.832) (end 29.222 -50.28) (width 0.25) (layer F.Cu) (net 8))
 (segment (start 30.222 -51.304) (end 31.75 -52.832) (width 0.25) (layer F.Cu) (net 10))
 (segment (start 30.222 -34.071) (end 30.222 -51.304) (width 0.25) (layer F.Cu) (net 10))
 (segment (start 31.222 -47.224) (end 31.222 -34.071) (width 0.25) (layer F.Cu) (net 12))
 (segment (start 36.83 -52.832) (end 31.222 -47.224) (width 0.25) (layer F.Cu) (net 12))
 (segment (start 41.91 -52.832) (end 32.19701 -43.11901) (width 0.25) (layer F.Cu) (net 14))
 (segment (start 32.222 -34.2625) (end 32.222 -34.071) (width 0.25) (layer F.Cu) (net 14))
 (segment (start 32.19701 -34.28749) (end 32.222 -34.2625) (width 0.25) (layer F.Cu) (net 14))
 (segment (start 32.19701 -43.11901) (end 32.19701 -34.28749) (width 0.25) (layer F.Cu) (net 14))
 (segment (start 27.722 -44.16) (end 27.722 -34.071) (width 0.25) (layer F.Cu) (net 4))
 (segment (start 19.05 -52.832) (end 27.722 -44.16) (width 0.25) (layer F.Cu) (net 4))
 (segment (start 27.3685 -58.2295) (end 25.0825 -55.9435) (width 0.25) (layer F.Cu) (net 4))
 (segment (start 22.1615 -55.9435) (end 19.05 -52.832) (width 0.25) (layer F.Cu) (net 4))
 (segment (start 25.0825 -55.9435) (end 22.1615 -55.9435) (width 0.25) (layer F.Cu) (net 4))
 (segment (start 28.722 -48.24) (end 28.722 -34.071) (width 0.25) (layer F.Cu) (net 7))
 (segment (start 24.13 -52.832) (end 28.722 -48.24) (width 0.25) (layer F.Cu) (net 7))
 (segment (start 29.722 -52.32) (end 29.722 -34.071) (width 0.25) (layer F.Cu) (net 9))
 (segment (start 29.21 -52.832) (end 29.722 -52.32) (width 0.25) (layer F.Cu) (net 9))
 (segment (start 33.489002 -52.832) (end 34.29 -52.832) (width 0.25) (layer F.Cu) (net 11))
 (segment (start 30.722 -50.064998) (end 33.489002 -52.832) (width 0.25) (layer F.Cu) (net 11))
 (segment (start 30.722 -34.071) (end 30.722 -50.064998) (width 0.25) (layer F.Cu) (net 11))
 (segment (start 31.722 -45.184) (end 39.37 -52.832) (width 0.25) (layer F.Cu) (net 13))
 (segment (start 31.722 -34.071) (end 31.722 -45.184) (width 0.25) (layer F.Cu) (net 13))
 (segment (start 32.722 -41.104) (end 44.45 -52.832) (width 0.25) (layer F.Cu) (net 1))
 (segment (start 32.722 -34.071) (end 32.722 -41.104) (width 0.25) (layer F.Cu) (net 1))
 (segment (start 39.0525 -58.2295) (end 34.9885 -58.2295) (width 0.25) (layer F.Cu) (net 1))
 (segment (start 44.45 -52.832) (end 39.0525 -58.2295) (width 0.25) (layer F.Cu) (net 1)))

